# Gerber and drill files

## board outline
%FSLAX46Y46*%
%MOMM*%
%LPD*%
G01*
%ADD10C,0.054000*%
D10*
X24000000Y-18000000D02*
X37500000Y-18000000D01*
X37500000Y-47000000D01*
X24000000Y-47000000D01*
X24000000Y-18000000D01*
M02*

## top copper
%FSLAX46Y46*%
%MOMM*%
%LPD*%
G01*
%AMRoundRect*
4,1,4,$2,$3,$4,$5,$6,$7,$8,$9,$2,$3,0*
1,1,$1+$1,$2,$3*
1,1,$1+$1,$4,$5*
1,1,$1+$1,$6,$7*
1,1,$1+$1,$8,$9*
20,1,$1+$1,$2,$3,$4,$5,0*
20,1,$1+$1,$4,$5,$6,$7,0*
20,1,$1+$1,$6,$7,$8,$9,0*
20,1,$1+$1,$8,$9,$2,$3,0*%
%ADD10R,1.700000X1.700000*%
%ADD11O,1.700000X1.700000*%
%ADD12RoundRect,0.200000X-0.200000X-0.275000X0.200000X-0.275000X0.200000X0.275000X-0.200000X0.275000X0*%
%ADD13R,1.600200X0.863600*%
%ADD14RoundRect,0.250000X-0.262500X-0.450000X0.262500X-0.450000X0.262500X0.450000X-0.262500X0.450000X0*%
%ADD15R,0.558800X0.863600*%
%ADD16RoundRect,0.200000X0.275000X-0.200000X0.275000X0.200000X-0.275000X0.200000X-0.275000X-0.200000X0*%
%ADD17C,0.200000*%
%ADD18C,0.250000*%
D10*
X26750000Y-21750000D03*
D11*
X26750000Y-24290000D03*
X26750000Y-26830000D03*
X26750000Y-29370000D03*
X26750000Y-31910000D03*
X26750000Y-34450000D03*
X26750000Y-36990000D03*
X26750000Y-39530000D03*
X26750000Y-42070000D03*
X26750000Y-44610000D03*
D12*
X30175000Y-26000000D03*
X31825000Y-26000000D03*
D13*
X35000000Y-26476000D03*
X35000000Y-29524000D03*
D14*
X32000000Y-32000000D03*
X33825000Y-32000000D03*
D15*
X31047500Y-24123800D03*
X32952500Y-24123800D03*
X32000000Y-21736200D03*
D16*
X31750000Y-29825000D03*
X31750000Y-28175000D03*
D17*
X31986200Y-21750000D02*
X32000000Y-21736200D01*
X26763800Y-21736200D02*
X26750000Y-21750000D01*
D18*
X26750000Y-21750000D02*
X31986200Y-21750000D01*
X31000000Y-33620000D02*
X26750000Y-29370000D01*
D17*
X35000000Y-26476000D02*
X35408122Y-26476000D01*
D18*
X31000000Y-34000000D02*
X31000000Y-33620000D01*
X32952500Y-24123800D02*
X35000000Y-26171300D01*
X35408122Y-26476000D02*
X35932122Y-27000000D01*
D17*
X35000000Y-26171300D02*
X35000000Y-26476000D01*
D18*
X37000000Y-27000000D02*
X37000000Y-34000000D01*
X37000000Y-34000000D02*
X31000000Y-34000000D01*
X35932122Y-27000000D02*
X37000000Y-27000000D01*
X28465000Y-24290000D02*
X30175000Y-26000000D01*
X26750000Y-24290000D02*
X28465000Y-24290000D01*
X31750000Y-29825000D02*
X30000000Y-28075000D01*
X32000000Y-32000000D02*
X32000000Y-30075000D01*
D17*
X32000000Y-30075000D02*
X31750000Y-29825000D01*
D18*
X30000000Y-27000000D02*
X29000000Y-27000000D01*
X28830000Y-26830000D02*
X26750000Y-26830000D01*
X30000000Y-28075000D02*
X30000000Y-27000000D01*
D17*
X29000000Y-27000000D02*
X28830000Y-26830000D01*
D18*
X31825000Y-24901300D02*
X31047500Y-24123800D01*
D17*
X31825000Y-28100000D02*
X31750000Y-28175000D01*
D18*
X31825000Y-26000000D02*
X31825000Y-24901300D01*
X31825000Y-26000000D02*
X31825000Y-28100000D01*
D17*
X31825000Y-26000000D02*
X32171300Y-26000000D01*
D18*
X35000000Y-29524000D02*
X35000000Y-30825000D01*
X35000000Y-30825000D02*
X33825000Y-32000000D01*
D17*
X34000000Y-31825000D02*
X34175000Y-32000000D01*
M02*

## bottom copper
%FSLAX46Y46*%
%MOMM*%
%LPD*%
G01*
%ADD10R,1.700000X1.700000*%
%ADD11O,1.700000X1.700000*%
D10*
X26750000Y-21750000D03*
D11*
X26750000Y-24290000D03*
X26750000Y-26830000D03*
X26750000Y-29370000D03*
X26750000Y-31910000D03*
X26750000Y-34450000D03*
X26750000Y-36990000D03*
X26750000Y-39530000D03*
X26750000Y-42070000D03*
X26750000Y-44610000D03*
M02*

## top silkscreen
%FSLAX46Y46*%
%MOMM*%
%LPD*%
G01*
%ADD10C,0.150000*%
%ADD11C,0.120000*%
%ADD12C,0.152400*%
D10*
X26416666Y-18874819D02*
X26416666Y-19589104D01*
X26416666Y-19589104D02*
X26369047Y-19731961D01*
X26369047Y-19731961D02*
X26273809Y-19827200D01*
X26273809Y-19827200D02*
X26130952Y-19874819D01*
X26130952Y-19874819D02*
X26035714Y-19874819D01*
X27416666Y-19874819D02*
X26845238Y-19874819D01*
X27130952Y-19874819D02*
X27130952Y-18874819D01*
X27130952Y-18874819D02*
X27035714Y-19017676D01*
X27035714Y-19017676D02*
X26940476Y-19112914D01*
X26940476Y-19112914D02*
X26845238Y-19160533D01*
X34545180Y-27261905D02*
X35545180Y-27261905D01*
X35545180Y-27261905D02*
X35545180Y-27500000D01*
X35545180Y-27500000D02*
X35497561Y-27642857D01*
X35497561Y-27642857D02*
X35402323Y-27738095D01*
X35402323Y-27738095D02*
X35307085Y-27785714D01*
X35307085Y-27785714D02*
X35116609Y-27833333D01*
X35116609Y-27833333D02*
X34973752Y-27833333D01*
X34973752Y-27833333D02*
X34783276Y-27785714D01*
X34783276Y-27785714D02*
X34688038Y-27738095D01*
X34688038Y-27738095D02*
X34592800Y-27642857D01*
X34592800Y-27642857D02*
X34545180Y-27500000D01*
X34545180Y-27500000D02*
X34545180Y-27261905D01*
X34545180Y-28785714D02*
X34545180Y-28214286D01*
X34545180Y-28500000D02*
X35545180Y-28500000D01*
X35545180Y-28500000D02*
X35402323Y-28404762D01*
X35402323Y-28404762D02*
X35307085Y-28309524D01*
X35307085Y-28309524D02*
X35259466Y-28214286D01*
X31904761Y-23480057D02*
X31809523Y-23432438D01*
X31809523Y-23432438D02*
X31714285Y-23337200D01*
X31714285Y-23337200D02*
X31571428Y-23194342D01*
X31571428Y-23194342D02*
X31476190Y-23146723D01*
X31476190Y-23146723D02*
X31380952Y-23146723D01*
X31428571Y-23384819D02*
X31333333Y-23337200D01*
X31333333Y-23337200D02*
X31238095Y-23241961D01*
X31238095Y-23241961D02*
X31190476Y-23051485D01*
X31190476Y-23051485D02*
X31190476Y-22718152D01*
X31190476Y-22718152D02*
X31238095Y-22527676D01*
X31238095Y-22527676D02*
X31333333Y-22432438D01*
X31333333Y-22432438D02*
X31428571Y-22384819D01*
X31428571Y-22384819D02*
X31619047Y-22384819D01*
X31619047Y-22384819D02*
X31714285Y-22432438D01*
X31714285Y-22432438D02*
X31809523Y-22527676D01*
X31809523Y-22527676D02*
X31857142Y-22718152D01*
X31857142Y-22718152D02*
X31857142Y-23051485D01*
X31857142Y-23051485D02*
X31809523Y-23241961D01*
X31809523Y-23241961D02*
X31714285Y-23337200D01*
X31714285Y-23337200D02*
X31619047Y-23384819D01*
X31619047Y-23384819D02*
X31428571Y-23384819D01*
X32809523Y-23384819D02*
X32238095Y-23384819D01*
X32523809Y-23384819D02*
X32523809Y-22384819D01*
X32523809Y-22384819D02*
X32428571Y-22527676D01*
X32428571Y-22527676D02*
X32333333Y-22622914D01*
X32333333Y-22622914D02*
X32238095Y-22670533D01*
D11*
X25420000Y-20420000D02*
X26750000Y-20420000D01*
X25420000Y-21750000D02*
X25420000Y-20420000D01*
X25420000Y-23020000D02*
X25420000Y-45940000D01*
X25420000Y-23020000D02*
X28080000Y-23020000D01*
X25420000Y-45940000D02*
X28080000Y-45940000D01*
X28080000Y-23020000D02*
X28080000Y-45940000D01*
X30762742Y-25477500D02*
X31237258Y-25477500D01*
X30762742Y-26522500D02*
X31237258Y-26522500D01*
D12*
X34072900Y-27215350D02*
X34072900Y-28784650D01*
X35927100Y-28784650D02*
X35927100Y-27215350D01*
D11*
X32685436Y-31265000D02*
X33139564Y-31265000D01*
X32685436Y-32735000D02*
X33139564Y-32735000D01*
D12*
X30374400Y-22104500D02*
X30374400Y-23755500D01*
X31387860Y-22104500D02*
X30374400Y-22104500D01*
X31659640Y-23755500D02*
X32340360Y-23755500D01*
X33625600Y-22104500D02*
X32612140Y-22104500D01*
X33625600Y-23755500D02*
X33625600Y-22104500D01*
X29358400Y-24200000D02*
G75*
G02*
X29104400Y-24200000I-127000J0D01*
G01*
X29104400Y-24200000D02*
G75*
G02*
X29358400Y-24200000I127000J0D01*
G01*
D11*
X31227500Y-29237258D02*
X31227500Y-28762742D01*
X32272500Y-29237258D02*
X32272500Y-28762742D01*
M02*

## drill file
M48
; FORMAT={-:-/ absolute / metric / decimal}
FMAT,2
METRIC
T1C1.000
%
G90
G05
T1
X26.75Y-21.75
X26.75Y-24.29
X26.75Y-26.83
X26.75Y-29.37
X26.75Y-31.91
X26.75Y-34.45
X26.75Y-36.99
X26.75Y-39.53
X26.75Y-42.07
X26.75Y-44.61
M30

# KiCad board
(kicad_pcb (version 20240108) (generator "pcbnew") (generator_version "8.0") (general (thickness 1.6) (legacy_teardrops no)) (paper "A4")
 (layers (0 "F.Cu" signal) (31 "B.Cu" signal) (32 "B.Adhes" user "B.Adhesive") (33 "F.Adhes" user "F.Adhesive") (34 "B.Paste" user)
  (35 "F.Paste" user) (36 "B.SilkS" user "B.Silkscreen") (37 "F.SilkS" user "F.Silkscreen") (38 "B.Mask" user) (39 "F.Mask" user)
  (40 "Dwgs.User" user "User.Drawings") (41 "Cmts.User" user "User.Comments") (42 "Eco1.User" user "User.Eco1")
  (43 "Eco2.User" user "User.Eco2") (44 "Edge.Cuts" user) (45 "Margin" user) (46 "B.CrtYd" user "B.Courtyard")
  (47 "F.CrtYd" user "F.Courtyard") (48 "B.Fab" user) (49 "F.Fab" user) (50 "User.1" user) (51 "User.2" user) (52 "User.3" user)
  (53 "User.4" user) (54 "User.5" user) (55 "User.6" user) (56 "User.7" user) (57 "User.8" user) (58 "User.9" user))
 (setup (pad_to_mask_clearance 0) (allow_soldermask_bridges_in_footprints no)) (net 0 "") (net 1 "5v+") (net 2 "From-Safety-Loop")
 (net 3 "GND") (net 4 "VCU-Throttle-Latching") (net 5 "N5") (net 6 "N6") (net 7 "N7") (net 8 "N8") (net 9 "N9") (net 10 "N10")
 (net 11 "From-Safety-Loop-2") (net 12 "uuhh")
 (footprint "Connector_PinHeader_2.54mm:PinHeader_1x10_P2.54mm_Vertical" (layer "F.Cu") (at 26.75 21.75)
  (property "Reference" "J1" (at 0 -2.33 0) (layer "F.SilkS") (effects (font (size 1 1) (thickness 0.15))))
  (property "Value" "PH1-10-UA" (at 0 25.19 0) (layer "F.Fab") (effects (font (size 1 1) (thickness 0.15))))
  (fp_line (start -1.33 -1.33) (end 0 -1.33) (stroke (width 0.12) (type solid)) (layer "F.SilkS"))
  (fp_line (start -1.33 0) (end -1.33 -1.33) (stroke (width 0.12) (type solid)) (layer "F.SilkS"))
  (fp_line (start -1.33 1.27) (end -1.33 24.19) (stroke (width 0.12) (type solid)) (layer "F.SilkS"))
  (fp_line (start -1.33 1.27) (end 1.33 1.27) (stroke (width 0.12) (type solid)) (layer "F.SilkS"))
  (fp_line (start -1.33 24.19) (end 1.33 24.19) (stroke (width 0.12) (type solid)) (layer "F.SilkS"))
  (fp_line (start 1.33 1.27) (end 1.33 24.19) (stroke (width 0.12) (type solid)) (layer "F.SilkS"))
  (pad "1" thru_hole rect (at 0 0) (size 1.7 1.7) (drill 1) (layers "*.Cu" "*.Mask") (remove_unused_layers no) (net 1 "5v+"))
  (pad "2" thru_hole oval (at 0 2.54) (size 1.7 1.7) (drill 1) (layers "*.Cu" "*.Mask") (remove_unused_layers no) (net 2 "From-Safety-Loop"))
  (pad "3" thru_hole oval (at 0 5.08) (size 1.7 1.7) (drill 1) (layers "*.Cu" "*.Mask") (remove_unused_layers no) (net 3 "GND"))
  (pad "4" thru_hole oval (at 0 7.62) (size 1.7 1.7) (drill 1) (layers "*.Cu" "*.Mask") (remove_unused_layers no)
   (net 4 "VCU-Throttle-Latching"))
  (pad "5" thru_hole oval (at 0 10.16) (size 1.7 1.7) (drill 1) (layers "*.Cu" "*.Mask") (remove_unused_layers no) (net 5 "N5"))
  (pad "6" thru_hole oval (at 0 12.7) (size 1.7 1.7) (drill 1) (layers "*.Cu" "*.Mask") (remove_unused_layers no) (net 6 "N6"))
  (pad "7" thru_hole oval (at 0 15.24) (size 1.7 1.7) (drill 1) (layers "*.Cu" "*.Mask") (remove_unused_layers no) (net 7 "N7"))
  (pad "8" thru_hole oval (at 0 17.78) (size 1.7 1.7) (drill 1) (layers "*.Cu" "*.Mask") (remove_unused_layers no) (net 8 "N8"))
  (pad "9" thru_hole oval (at 0 20.32) (size 1.7 1.7) (drill 1) (layers "*.Cu" "*.Mask") (remove_unused_layers no) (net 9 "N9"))
  (pad "10" thru_hole oval (at 0 22.86) (size 1.7 1.7) (drill 1) (layers "*.Cu" "*.Mask") (remove_unused_layers no) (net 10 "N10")))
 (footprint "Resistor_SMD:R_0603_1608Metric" (layer "F.Cu") (at 31 26)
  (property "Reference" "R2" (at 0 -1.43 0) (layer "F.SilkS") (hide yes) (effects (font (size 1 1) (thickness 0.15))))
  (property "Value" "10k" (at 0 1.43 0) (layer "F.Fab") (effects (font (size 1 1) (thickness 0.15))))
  (fp_line (start -0.237258 -0.5225) (end 0.237258 -0.5225) (stroke (width 0.12) (type solid)) (layer "F.SilkS"))
  (fp_line (start -0.237258 0.5225) (end 0.237258 0.5225) (stroke (width 0.12) (type solid)) (layer "F.SilkS"))
  (pad "1" smd roundrect (at -0.825 0) (size 0.8 0.95) (layers "F.Cu" "F.Paste" "F.Mask") (roundrect_rratio 0.25) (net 2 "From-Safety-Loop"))
  (pad "2" smd roundrect (at 0.825 0) (size 0.8 0.95) (layers "F.Cu" "F.Paste" "F.Mask") (roundrect_rratio 0.25)
   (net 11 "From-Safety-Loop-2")))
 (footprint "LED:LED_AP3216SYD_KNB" (layer "F.Cu") (at 35 28 -90)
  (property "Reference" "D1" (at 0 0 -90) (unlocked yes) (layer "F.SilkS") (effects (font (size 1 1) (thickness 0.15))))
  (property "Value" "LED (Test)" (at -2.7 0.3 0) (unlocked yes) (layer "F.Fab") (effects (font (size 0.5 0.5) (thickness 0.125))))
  (fp_line (start -0.78465 0.9271) (end 0.78465 0.9271) (stroke (width 0.1524) (type solid)) (layer "F.SilkS"))
  (fp_line (start 0.78465 -0.9271) (end -0.78465 -0.9271) (stroke (width 0.1524) (type solid)) (layer "F.SilkS"))
  (pad "1" smd rect (at -1.524 0 270) (size 0.8636 1.6002) (layers "F.Cu" "F.Paste" "F.Mask") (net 4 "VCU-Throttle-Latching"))
  (pad "2" smd rect (at 1.524 0 270) (size 0.8636 1.6002) (layers "F.Cu" "F.Paste" "F.Mask") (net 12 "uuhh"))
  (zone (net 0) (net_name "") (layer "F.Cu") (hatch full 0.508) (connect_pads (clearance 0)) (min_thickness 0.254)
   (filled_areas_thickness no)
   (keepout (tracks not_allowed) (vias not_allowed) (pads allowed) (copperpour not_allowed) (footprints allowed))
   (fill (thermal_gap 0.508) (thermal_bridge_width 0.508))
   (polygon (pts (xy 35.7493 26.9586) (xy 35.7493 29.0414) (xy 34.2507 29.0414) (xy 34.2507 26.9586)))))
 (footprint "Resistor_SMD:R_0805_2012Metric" (layer "F.Cu") (at 32.9125 32)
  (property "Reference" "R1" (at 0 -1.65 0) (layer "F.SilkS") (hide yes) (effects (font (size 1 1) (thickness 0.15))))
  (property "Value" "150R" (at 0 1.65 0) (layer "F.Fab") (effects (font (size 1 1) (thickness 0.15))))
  (fp_line (start -0.227064 -0.735) (end 0.227064 -0.735) (stroke (width 0.12) (type solid)) (layer "F.SilkS"))
  (fp_line (start -0.227064 0.735) (end 0.227064 0.735) (stroke (width 0.12) (type solid)) (layer "F.SilkS"))
  (pad "1" smd roundrect (at -0.9125 0) (size 1.025 1.4) (layers "F.Cu" "F.Paste" "F.Mask") (roundrect_rratio 0.243902) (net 3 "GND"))
  (pad "2" smd roundrect (at 0.9125 0) (size 1.025 1.4) (layers "F.Cu" "F.Paste" "F.Mask") (roundrect_rratio 0.243902) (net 12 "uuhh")))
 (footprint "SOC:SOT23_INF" (layer "F.Cu") (at 32 22.93)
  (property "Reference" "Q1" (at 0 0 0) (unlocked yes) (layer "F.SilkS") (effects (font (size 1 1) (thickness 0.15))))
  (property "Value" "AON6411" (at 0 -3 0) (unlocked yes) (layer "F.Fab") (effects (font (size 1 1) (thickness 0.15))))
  (fp_line (start -1.6256 -0.8255) (end -1.6256 0.8255) (stroke (width 0.1524) (type solid)) (layer "F.SilkS"))
  (fp_line (start -0.61214 -0.8255) (end -1.6256 -0.8255) (stroke (width 0.1524) (type solid)) (layer "F.SilkS"))
  (fp_line (start -0.34036 0.8255) (end 0.34036 0.8255) (stroke (width 0.1524) (type solid)) (layer "F.SilkS"))
  (fp_line (start 1.6256 -0.8255) (end 0.61214 -0.8255) (stroke (width 0.1524) (type solid)) (layer "F.SilkS"))
  (fp_line (start 1.6256 0.8255) (end 1.6256 -0.8255) (stroke (width 0.1524) (type solid)) (layer "F.SilkS"))
  (fp_circle (center -2.7686 1.27) (end -2.6416 1.27) (stroke (width 0.1524) (type solid)) (fill none) (layer "F.SilkS"))
  (pad "1" smd rect (at -0.9525 1.1938) (size 0.5588 0.8636) (layers "F.Cu" "F.Paste" "F.Mask") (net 11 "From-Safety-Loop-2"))
  (pad "2" smd rect (at 0.9525 1.1938) (size 0.5588 0.8636) (layers "F.Cu" "F.Paste" "F.Mask") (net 4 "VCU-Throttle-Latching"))
  (pad "3" smd rect (at 0 -1.1938) (size 0.5588 0.8636) (layers "F.Cu" "F.Paste" "F.Mask") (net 1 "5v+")))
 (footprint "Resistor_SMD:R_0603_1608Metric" (layer "F.Cu") (at 31.75 29 90)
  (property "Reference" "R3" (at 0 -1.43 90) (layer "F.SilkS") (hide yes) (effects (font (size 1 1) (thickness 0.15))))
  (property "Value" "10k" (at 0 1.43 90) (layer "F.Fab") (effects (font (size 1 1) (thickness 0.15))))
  (fp_line (start -0.237258 -0.5225) (end 0.237258 -0.5225) (stroke (width 0.12) (type solid)) (layer "F.SilkS"))
  (fp_line (start -0.237258 0.5225) (end 0.237258 0.5225) (stroke (width 0.12) (type solid)) (layer "F.SilkS"))
  (pad "1" smd roundrect (at -0.825 0 90) (size 0.8 0.95) (layers "F.Cu" "F.Paste" "F.Mask") (roundrect_rratio 0.25) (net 3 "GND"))
  (pad "2" smd roundrect (at 0.825 0 90) (size 0.8 0.95) (layers "F.Cu" "F.Paste" "F.Mask") (roundrect_rratio 0.25)
   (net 11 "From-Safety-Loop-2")))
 (gr_rect (start 24 18) (end 37.5 47) (stroke (width 0.054) (type default)) (fill none) (layer "Edge.Cuts"))
 (segment (start 31.9862 21.75) (end 32 21.7362) (width 0.2) (layer "F.Cu") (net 1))
 (segment (start 26.7638 21.7362) (end 26.75 21.75) (width 0.2) (layer "F.Cu") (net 1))
 (segment (start 26.75 21.75) (end 31.9862 21.75) (width 0.25) (layer "F.Cu") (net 1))
 (segment (start 31 33.62) (end 26.75 29.37) (width 0.25) (layer "F.Cu") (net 4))
 (segment (start 35 26.476) (end 35.408122 26.476) (width 0.2) (layer "F.Cu") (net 4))
 (segment (start 31 34) (end 31 33.62) (width 0.25) (layer "F.Cu") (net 4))
 (segment (start 32.9525 24.1238) (end 35 26.1713) (width 0.25) (layer "F.Cu") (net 4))
 (segment (start 35.408122 26.476) (end 35.932122 27) (width 0.25) (layer "F.Cu") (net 4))
 (segment (start 35 26.1713) (end 35 26.476) (width 0.2) (layer "F.Cu") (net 4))
 (segment (start 37 27) (end 37 34) (width 0.25) (layer "F.Cu") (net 4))
 (segment (start 37 34) (end 31 34) (width 0.25) (layer "F.Cu") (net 4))
 (segment (start 35.932122 27) (end 37 27) (width 0.25) (layer "F.Cu") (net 4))
 (segment (start 28.465 24.29) (end 30.175 26) (width 0.25) (layer "F.Cu") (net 2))
 (segment (start 26.75 24.29) (end 28.465 24.29) (width 0.25) (layer "F.Cu") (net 2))
 (segment (start 31.75 29.825) (end 30 28.075) (width 0.25) (layer "F.Cu") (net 3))
 (segment (start 32 32) (end 32 30.075) (width 0.25) (layer "F.Cu") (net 3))
 (segment (start 32 30.075) (end 31.75 29.825) (width 0.2) (layer "F.Cu") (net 3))
 (segment (start 30 27) (end 29 27) (width 0.25) (layer "F.Cu") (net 3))
 (segment (start 28.83 26.83) (end 26.75 26.83) (width 0.25) (layer "F.Cu") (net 3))
 (segment (start 30 28.075) (end 30 27) (width 0.25) (layer "F.Cu") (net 3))
 (segment (start 29 27) (end 28.83 26.83) (width 0.2) (layer "F.Cu") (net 3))
 (segment (start 31.825 24.9013) (end 31.0475 24.1238) (width 0.25) (layer "F.Cu") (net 11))
 (segment (start 31.825 28.1) (end 31.75 28.175) (width 0.2) (layer "F.Cu") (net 11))
 (segment (start 31.825 26) (end 31.825 24.9013) (width 0.25) (layer "F.Cu") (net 11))
 (segment (start 31.825 26) (end 31.825 28.1) (width 0.25) (layer "F.Cu") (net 11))
 (segment (start 31.825 26) (end 32.1713 26) (width 0.2) (layer "F.Cu") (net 11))
 (segment (start 35 29.524) (end 35 30.825) (width 0.25) (layer "F.Cu") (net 12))
 (segment (start 35 30.825) (end 33.825 32) (width 0.25) (layer "F.Cu") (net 12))
 (segment (start 34 31.825) (end 34.175 32) (width 0.2) (layer "F.Cu") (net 12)))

